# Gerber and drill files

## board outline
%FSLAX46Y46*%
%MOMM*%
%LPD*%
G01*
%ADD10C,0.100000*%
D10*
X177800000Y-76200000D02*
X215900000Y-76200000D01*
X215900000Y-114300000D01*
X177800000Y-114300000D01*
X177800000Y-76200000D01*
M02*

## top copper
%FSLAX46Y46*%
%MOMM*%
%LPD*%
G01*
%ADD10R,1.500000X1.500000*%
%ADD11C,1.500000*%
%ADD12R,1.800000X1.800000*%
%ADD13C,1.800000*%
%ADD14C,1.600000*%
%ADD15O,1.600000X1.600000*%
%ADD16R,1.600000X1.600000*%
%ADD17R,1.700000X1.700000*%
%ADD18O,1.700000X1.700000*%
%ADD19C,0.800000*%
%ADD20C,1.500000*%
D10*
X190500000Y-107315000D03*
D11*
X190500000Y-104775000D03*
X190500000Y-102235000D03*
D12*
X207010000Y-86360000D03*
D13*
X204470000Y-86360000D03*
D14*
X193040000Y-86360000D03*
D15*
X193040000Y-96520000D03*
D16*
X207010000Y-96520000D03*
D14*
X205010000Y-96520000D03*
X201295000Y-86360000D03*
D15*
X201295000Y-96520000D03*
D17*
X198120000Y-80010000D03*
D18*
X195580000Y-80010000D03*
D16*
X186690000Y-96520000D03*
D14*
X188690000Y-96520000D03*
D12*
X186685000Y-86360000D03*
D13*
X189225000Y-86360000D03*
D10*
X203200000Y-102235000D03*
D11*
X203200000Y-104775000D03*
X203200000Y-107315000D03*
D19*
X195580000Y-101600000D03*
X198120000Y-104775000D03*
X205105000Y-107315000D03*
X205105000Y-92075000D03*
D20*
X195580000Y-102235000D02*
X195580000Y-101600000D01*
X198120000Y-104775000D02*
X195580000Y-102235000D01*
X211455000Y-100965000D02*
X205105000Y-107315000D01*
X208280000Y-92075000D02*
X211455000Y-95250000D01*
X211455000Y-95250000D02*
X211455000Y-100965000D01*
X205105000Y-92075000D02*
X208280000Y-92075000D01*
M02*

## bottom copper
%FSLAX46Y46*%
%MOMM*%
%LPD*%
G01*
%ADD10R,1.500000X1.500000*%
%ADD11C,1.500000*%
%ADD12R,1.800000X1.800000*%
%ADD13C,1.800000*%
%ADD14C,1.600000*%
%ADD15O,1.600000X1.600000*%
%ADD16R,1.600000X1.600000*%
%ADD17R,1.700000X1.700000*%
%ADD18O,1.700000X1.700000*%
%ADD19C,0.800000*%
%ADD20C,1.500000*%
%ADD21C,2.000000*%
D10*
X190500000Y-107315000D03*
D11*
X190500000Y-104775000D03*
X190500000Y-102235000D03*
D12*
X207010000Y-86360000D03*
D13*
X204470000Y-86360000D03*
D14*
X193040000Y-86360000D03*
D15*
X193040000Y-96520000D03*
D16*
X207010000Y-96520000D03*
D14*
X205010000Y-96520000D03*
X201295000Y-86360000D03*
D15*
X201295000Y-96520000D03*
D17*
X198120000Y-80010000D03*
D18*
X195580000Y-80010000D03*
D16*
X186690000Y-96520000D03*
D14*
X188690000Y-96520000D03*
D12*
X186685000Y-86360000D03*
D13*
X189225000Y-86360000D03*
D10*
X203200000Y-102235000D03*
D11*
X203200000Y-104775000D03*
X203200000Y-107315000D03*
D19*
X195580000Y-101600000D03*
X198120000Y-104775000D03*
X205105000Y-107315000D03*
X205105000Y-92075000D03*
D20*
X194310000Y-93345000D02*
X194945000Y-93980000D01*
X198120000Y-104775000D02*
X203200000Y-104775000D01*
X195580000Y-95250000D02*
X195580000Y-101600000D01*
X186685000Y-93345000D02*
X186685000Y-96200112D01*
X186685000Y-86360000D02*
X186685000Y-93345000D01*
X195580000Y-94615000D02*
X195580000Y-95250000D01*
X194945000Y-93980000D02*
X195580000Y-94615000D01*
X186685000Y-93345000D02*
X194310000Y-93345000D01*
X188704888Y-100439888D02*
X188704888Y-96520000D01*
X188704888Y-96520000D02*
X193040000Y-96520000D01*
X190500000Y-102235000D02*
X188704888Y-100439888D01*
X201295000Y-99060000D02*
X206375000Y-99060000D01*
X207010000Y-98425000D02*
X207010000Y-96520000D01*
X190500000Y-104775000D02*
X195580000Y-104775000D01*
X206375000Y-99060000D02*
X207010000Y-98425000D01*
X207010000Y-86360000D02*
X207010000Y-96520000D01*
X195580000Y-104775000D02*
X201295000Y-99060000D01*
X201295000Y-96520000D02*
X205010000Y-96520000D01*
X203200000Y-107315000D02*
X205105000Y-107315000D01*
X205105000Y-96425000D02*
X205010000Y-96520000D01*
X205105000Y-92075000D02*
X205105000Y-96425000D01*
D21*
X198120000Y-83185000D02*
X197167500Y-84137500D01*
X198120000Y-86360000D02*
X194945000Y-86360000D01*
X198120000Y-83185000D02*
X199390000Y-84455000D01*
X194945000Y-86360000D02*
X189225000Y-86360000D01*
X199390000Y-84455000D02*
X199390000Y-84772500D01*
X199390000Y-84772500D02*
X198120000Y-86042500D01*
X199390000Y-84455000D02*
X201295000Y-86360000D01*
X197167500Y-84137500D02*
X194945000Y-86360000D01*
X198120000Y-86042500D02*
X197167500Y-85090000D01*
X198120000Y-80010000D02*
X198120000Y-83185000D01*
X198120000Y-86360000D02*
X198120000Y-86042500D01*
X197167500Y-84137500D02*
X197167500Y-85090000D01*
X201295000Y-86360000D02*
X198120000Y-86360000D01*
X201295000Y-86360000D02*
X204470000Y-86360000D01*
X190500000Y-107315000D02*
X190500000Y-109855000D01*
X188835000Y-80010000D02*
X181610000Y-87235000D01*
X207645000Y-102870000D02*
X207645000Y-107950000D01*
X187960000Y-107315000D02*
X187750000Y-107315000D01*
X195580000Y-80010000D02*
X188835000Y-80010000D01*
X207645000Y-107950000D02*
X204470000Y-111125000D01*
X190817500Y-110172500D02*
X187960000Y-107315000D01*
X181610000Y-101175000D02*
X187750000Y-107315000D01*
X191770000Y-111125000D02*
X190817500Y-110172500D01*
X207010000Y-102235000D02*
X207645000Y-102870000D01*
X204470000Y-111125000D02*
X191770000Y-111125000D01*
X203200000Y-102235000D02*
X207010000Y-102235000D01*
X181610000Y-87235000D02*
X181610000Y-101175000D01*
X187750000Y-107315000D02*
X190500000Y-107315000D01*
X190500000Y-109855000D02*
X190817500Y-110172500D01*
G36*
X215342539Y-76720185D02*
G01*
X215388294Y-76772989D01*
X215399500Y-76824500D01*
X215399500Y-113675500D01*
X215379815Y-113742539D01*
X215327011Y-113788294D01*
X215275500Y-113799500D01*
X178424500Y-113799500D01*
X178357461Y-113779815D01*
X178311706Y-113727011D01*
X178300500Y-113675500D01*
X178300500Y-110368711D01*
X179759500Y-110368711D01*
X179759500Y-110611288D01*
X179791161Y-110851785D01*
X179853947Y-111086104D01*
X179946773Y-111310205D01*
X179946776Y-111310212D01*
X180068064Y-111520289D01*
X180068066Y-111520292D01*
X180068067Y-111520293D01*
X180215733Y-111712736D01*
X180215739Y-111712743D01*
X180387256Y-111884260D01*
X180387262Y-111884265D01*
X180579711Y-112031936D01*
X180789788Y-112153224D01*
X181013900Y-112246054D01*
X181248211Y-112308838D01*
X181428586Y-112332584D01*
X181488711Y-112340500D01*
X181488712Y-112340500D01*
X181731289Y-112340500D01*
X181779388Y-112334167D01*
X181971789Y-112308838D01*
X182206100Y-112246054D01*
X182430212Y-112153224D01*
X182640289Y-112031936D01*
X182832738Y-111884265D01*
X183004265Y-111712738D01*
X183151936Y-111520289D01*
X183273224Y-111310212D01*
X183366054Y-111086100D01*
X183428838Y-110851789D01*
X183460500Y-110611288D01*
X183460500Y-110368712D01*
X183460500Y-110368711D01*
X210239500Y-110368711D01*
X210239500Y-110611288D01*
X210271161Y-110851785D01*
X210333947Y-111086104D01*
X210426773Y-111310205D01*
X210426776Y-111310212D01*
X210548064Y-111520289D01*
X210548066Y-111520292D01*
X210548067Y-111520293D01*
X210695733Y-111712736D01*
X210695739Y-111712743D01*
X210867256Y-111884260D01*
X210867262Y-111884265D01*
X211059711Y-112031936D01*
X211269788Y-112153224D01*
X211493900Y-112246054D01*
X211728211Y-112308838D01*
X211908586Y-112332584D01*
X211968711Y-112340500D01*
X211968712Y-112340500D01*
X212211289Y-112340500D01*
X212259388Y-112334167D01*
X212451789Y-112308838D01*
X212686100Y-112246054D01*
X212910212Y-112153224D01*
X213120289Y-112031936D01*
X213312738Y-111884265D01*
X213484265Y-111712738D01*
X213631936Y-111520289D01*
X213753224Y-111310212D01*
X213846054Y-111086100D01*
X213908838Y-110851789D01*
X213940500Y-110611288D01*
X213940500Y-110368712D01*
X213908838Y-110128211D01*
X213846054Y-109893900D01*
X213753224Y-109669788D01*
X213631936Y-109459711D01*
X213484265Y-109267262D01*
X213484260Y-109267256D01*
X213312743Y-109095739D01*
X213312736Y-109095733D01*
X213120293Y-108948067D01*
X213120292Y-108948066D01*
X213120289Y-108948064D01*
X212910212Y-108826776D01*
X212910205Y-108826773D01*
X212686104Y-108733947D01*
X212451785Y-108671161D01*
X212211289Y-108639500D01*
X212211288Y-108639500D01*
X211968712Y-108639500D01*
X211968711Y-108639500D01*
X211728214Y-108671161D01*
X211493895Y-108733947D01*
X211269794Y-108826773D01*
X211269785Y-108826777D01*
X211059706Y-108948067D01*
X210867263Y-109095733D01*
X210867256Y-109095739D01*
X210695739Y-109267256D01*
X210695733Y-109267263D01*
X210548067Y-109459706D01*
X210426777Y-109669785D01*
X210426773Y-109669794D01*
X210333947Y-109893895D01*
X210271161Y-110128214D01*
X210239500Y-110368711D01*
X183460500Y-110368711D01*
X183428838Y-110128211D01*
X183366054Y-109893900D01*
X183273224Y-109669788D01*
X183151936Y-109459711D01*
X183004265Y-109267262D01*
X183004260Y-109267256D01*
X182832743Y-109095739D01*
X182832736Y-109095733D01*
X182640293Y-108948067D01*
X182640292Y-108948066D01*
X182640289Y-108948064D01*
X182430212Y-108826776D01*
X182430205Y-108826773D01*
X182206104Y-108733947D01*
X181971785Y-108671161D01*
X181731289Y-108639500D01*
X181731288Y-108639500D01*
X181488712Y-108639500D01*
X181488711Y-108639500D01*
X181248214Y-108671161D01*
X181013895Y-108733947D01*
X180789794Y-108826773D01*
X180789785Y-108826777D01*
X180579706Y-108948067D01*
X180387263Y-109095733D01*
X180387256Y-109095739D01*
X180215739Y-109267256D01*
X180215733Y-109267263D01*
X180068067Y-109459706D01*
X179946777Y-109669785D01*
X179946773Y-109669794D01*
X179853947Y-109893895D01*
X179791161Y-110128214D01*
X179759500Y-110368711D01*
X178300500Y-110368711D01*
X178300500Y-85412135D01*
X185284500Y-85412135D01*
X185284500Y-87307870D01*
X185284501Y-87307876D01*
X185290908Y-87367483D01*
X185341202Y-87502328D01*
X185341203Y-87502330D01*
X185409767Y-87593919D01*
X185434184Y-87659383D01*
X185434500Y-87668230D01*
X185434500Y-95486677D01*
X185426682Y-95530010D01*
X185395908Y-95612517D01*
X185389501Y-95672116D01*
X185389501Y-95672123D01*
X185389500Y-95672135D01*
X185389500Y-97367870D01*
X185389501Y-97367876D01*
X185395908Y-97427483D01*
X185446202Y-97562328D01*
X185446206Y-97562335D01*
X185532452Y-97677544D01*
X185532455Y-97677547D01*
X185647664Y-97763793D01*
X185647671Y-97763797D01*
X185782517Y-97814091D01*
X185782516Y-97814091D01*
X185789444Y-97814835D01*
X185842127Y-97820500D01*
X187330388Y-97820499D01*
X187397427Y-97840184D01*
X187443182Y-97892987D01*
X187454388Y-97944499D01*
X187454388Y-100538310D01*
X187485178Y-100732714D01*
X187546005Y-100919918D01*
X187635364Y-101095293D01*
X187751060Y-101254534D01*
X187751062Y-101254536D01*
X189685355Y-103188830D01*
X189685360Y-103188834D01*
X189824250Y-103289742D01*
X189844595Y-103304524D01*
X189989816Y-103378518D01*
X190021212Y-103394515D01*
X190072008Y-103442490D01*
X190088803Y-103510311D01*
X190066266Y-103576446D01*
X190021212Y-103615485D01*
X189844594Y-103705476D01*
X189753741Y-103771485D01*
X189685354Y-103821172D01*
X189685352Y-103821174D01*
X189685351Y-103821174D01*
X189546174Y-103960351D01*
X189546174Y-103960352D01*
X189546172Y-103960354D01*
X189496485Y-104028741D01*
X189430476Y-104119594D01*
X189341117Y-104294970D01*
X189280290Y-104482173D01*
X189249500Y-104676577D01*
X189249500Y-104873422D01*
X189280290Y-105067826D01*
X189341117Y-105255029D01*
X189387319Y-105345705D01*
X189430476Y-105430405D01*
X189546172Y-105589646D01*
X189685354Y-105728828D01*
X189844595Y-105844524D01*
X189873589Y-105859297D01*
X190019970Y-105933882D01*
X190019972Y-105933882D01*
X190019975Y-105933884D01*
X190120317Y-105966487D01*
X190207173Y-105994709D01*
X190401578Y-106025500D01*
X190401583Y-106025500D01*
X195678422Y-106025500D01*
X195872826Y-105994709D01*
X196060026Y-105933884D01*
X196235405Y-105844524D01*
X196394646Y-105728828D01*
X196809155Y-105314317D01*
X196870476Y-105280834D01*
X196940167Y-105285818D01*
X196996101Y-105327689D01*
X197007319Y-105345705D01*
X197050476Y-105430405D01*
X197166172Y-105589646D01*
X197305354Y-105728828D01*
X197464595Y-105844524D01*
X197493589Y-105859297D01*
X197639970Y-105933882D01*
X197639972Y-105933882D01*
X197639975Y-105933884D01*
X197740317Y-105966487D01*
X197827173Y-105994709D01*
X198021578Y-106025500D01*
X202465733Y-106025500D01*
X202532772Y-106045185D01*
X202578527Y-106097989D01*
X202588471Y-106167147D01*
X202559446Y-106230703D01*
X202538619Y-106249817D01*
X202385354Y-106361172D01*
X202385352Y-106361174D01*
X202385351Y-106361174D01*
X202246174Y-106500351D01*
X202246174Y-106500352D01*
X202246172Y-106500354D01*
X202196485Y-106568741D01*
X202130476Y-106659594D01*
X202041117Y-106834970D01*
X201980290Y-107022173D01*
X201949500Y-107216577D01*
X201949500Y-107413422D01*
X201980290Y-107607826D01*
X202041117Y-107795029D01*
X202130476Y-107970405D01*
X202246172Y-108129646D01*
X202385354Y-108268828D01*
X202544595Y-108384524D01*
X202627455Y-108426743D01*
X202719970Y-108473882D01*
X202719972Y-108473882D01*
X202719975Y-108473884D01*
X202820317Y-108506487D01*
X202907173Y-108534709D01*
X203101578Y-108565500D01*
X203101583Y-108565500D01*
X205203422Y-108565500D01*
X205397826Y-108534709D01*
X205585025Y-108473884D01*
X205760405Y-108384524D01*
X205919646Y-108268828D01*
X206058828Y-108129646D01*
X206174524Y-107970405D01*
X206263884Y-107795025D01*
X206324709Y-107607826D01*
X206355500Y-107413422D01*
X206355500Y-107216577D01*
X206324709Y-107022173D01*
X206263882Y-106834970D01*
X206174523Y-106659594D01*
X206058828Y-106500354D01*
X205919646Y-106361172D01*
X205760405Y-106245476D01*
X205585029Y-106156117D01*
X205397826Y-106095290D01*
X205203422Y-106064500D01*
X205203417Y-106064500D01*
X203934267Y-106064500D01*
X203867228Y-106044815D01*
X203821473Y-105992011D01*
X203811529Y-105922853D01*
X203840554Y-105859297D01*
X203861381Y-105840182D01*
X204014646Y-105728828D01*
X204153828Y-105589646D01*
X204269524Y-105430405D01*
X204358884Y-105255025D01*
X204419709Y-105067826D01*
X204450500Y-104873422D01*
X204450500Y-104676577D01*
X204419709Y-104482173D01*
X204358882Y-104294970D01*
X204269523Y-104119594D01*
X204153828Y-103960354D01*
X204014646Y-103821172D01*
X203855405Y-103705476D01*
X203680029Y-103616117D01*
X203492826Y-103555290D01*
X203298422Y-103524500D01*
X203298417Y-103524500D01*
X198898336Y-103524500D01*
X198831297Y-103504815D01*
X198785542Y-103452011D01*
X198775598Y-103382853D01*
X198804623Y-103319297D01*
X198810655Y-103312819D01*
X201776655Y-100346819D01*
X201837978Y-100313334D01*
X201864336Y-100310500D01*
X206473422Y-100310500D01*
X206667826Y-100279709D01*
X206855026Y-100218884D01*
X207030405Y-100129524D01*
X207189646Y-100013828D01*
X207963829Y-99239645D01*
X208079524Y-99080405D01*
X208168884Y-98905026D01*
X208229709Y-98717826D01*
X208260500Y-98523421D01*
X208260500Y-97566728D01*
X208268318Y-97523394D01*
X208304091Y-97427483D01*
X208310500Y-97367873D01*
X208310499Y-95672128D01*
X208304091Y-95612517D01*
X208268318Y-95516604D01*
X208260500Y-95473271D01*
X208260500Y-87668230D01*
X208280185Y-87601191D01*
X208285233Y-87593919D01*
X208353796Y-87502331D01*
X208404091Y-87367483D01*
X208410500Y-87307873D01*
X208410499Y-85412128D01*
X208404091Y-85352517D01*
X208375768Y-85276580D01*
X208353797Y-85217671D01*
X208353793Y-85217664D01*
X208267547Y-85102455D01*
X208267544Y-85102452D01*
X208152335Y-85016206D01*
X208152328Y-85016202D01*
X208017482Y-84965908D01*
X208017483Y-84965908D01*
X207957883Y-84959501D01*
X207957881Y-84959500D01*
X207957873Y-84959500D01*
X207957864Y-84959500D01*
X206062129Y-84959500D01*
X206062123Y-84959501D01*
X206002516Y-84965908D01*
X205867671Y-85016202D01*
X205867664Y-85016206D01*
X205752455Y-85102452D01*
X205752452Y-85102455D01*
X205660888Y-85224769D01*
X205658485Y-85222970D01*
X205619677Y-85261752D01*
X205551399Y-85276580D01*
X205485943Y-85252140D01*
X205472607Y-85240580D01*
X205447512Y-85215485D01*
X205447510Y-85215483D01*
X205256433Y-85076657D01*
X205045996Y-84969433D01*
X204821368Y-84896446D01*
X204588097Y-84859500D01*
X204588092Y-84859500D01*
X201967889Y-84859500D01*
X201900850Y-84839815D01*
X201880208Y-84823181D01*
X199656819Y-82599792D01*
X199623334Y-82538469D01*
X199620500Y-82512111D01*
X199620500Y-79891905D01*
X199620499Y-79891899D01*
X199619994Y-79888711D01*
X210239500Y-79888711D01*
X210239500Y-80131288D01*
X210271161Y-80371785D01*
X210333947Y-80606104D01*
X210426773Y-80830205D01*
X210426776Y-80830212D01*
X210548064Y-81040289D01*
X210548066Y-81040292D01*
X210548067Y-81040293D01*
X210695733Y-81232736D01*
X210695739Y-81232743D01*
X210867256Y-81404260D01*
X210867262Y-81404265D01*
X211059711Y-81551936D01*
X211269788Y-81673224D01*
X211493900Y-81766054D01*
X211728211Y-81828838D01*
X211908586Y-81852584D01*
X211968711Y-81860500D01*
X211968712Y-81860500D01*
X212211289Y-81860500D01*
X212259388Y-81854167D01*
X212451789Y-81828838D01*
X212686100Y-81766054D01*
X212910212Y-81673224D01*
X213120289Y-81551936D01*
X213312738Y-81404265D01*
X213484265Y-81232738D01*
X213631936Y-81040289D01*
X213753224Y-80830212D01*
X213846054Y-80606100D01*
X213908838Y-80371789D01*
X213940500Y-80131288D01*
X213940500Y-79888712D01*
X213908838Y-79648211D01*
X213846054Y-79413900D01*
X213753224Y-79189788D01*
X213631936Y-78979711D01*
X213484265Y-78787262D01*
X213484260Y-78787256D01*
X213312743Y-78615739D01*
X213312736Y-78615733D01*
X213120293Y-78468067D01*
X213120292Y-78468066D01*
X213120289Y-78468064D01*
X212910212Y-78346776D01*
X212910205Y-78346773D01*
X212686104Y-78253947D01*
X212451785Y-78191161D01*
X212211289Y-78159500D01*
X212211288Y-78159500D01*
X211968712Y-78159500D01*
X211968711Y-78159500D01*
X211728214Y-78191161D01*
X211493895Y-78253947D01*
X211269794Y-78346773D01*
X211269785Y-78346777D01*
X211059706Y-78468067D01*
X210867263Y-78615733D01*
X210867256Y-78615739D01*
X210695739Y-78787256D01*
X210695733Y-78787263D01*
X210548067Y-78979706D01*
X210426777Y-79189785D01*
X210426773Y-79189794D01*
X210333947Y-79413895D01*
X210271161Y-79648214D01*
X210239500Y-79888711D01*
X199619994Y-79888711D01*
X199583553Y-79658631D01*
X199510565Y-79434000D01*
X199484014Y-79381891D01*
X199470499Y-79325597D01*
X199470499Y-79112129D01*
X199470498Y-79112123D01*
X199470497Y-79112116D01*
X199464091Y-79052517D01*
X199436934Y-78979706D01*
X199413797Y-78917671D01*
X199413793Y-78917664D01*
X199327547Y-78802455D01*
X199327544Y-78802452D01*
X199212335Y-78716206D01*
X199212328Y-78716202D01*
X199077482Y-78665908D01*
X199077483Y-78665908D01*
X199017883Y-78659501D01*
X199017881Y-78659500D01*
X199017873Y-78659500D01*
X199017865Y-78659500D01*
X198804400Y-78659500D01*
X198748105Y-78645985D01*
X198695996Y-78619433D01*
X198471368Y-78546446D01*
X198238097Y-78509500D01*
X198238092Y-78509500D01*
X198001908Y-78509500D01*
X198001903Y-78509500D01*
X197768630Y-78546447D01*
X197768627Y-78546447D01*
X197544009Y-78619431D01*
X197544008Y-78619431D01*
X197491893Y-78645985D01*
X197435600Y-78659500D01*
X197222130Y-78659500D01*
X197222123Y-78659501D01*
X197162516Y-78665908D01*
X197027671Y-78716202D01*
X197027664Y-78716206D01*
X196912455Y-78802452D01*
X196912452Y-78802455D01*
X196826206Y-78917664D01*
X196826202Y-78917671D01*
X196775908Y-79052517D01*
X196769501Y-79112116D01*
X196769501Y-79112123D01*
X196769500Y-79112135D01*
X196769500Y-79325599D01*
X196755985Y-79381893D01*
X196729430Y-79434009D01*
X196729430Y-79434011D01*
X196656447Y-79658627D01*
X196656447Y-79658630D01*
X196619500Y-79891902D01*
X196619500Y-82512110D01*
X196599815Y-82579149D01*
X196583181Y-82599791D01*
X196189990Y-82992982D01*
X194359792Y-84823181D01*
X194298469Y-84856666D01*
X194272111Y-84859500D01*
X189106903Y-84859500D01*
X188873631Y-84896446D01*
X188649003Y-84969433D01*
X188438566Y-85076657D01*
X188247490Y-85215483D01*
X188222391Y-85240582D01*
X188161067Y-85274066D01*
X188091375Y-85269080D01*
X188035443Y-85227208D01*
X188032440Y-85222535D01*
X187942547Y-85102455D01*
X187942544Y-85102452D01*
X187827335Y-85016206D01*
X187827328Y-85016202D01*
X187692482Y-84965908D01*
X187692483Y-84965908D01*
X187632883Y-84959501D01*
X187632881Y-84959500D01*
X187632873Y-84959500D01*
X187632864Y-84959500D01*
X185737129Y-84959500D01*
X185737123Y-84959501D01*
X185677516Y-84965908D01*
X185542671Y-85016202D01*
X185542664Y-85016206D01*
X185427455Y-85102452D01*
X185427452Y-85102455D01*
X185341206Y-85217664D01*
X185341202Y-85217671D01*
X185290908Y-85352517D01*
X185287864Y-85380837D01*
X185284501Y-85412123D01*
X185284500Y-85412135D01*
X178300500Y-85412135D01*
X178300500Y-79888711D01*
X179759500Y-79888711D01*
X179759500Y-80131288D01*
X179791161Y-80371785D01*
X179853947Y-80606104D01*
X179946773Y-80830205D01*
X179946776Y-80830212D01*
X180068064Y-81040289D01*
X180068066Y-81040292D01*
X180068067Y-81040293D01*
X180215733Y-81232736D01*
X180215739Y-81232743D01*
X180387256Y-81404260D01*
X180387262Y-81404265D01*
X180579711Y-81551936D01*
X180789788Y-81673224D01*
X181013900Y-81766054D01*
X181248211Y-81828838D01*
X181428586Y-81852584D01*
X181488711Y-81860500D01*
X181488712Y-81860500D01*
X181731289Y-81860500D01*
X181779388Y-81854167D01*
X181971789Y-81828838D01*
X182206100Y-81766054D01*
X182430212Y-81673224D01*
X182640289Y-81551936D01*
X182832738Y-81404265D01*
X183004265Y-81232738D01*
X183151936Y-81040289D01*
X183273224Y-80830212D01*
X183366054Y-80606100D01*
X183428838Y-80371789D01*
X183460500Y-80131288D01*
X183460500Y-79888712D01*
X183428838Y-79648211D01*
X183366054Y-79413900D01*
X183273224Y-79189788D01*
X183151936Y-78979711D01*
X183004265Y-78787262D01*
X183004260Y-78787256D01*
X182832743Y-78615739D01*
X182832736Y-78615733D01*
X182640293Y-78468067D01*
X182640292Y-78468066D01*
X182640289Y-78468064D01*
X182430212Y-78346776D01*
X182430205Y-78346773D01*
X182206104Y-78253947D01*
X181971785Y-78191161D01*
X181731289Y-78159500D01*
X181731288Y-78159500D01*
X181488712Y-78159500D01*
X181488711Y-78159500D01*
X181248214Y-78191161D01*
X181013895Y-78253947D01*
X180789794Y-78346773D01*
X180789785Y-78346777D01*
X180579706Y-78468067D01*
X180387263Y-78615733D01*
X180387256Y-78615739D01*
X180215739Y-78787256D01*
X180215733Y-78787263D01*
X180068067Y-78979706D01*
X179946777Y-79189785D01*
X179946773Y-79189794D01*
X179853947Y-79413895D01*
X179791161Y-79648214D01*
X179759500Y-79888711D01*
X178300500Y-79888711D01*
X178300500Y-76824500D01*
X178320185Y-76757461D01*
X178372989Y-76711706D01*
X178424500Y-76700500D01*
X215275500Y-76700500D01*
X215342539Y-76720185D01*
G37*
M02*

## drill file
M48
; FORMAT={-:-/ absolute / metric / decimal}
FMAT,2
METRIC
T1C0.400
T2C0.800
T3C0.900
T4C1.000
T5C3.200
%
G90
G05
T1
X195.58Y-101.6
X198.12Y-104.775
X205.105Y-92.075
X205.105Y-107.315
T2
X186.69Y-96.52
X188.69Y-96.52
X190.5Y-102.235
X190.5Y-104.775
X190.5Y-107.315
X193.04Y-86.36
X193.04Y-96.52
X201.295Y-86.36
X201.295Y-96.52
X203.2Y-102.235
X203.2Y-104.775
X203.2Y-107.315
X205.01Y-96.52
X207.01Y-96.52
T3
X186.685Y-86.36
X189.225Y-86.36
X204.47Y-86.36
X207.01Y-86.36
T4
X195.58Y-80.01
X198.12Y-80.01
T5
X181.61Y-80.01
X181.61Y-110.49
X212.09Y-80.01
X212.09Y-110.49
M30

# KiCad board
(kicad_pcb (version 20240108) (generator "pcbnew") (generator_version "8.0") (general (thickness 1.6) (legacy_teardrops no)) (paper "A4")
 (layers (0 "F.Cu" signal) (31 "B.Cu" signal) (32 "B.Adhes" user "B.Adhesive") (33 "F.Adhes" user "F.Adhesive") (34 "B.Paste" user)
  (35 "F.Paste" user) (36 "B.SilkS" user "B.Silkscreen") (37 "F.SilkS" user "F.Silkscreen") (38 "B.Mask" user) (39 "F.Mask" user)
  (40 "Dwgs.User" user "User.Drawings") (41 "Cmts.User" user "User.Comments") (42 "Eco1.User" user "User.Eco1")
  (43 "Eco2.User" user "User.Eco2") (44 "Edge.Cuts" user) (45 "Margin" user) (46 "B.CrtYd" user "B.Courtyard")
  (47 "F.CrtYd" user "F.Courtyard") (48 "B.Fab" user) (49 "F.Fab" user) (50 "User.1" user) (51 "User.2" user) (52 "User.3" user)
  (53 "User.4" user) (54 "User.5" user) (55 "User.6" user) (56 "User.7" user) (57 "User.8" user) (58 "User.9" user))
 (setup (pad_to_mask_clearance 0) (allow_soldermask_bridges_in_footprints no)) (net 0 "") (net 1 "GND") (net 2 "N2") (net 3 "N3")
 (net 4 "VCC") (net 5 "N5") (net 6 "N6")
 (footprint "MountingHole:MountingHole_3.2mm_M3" (layer "F.Cu") (at 181.61 110.49)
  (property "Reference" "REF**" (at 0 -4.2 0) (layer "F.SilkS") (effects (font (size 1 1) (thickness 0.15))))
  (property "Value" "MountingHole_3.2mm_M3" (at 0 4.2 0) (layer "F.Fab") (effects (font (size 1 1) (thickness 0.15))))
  (pad "" np_thru_hole circle (at 0 0) (size 3.2 3.2) (drill 3.2) (layers "F&B.Cu" "*.Mask")))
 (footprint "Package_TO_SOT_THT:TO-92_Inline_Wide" (layer "F.Cu") (at 190.5 107.315 90)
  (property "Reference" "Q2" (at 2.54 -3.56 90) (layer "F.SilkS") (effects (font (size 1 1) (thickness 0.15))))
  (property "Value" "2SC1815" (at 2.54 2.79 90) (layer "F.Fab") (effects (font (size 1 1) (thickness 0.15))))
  (pad "1" thru_hole rect (at 0 0 90) (size 1.5 1.5) (drill 0.8) (layers "*.Cu" "*.Mask") (remove_unused_layers no) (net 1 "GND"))
  (pad "2" thru_hole circle (at 2.54 0 90) (size 1.5 1.5) (drill 0.8) (layers "*.Cu" "*.Mask") (remove_unused_layers no) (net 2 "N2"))
  (pad "3" thru_hole circle (at 5.08 0 90) (size 1.5 1.5) (drill 0.8) (layers "*.Cu" "*.Mask") (remove_unused_layers no) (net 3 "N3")))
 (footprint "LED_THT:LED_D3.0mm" (layer "F.Cu") (at 207.01 86.36 180)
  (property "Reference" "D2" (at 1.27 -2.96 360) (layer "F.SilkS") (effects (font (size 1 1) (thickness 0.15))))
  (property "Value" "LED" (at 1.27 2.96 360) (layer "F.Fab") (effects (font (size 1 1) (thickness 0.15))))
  (pad "1" thru_hole rect (at 0 0 180) (size 1.8 1.8) (drill 0.9) (layers "*.Cu" "*.Mask") (remove_unused_layers no) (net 2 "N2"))
  (pad "2" thru_hole circle (at 2.54 0 180) (size 1.8 1.8) (drill 0.9) (layers "*.Cu" "*.Mask") (remove_unused_layers no) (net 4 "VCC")))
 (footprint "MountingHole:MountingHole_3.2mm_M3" (layer "F.Cu") (at 212.09 110.49)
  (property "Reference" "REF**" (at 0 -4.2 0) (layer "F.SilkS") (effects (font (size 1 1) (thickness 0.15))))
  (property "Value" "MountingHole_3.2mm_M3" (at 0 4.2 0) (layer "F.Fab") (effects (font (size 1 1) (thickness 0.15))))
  (pad "" np_thru_hole circle (at 0 0) (size 3.2 3.2) (drill 3.2) (layers "F&B.Cu" "*.Mask")))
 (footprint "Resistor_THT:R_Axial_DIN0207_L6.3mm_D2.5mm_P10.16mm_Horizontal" (layer "F.Cu") (at 193.04 86.36 -90)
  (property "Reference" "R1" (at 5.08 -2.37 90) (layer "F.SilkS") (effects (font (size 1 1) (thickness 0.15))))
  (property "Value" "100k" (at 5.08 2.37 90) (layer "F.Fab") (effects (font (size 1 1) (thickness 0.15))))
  (pad "1" thru_hole circle (at 0 0 270) (size 1.6 1.6) (drill 0.8) (layers "*.Cu" "*.Mask") (remove_unused_layers no) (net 4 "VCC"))
  (pad "2" thru_hole oval (at 10.16 0 270) (size 1.6 1.6) (drill 0.8) (layers "*.Cu" "*.Mask") (remove_unused_layers no) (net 3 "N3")))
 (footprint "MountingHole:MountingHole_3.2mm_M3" (layer "F.Cu") (at 181.61 80.01)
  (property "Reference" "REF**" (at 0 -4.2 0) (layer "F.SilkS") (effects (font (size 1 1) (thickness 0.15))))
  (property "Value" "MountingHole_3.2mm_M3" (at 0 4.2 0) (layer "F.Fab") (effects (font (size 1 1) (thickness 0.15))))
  (pad "" np_thru_hole circle (at 0 0) (size 3.2 3.2) (drill 3.2) (layers "*.Cu" "*.Mask")))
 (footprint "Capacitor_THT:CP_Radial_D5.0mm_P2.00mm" (layer "F.Cu") (at 207.01 96.52 180)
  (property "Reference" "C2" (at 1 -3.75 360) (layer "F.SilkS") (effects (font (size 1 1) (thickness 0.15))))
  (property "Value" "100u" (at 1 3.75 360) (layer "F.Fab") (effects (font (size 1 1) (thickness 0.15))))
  (pad "1" thru_hole rect (at 0 0 180) (size 1.6 1.6) (drill 0.8) (layers "*.Cu" "*.Mask") (remove_unused_layers no) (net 2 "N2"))
  (pad "2" thru_hole circle (at 2 0 180) (size 1.6 1.6) (drill 0.8) (layers "*.Cu" "*.Mask") (remove_unused_layers no) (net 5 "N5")))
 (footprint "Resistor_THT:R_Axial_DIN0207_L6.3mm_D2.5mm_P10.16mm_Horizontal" (layer "F.Cu") (at 201.295 86.36 -90)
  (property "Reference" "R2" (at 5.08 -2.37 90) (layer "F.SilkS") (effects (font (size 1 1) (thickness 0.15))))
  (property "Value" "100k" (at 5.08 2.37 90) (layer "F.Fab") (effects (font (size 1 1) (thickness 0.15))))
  (pad "1" thru_hole circle (at 0 0 270) (size 1.6 1.6) (drill 0.8) (layers "*.Cu" "*.Mask") (remove_unused_layers no) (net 4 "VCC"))
  (pad "2" thru_hole oval (at 10.16 0 270) (size 1.6 1.6) (drill 0.8) (layers "*.Cu" "*.Mask") (remove_unused_layers no) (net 5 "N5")))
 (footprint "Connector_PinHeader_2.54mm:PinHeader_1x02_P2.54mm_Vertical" (layer "F.Cu") (at 198.12 80.01 -90)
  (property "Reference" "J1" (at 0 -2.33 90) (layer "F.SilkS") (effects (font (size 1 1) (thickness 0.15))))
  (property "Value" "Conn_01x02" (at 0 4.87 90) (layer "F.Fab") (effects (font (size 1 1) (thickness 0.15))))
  (pad "1" thru_hole rect (at 0 0 270) (size 1.7 1.7) (drill 1) (layers "*.Cu" "*.Mask") (remove_unused_layers no) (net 4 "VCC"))
  (pad "2" thru_hole oval (at 0 2.54 270) (size 1.7 1.7) (drill 1) (layers "*.Cu" "*.Mask") (remove_unused_layers no) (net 1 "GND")))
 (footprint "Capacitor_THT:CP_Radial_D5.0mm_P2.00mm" (layer "F.Cu") (at 186.69 96.52)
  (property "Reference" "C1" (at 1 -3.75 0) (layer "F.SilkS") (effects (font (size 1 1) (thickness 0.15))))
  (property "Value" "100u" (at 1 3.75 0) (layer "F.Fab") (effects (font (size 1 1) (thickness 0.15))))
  (pad "1" thru_hole rect (at 0 0) (size 1.6 1.6) (drill 0.8) (layers "*.Cu" "*.Mask") (remove_unused_layers no) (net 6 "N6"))
  (pad "2" thru_hole circle (at 2 0) (size 1.6 1.6) (drill 0.8) (layers "*.Cu" "*.Mask") (remove_unused_layers no) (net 3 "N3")))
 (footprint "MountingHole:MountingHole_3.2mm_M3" (layer "F.Cu") (at 212.09 80.01)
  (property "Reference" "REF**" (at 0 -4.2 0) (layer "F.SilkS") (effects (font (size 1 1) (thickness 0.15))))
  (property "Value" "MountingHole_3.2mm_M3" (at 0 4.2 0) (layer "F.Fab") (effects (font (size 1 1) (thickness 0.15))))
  (pad "" np_thru_hole circle (at 0 0) (size 3.2 3.2) (drill 3.2) (layers "F&B.Cu" "*.Mask")))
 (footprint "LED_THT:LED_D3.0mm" (layer "F.Cu") (at 186.685 86.36)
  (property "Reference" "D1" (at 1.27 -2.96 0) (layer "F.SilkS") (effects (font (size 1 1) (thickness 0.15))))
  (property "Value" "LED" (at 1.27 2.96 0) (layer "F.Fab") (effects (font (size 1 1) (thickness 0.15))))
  (pad "1" thru_hole rect (at 0 0) (size 1.8 1.8) (drill 0.9) (layers "*.Cu" "*.Mask") (remove_unused_layers no) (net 6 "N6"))
  (pad "2" thru_hole circle (at 2.54 0) (size 1.8 1.8) (drill 0.9) (layers "*.Cu" "*.Mask") (remove_unused_layers no) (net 4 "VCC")))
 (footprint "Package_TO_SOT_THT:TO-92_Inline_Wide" (layer "F.Cu") (at 203.2 102.235 -90)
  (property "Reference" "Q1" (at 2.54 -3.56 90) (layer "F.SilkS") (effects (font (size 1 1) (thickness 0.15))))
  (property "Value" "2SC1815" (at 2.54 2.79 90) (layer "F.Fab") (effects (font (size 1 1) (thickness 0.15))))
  (pad "1" thru_hole rect (at 0 0 270) (size 1.5 1.5) (drill 0.8) (layers "*.Cu" "*.Mask") (remove_unused_layers no) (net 1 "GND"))
  (pad "2" thru_hole circle (at 2.54 0 270) (size 1.5 1.5) (drill 0.8) (layers "*.Cu" "*.Mask") (remove_unused_layers no) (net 6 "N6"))
  (pad "3" thru_hole circle (at 5.08 0 270) (size 1.5 1.5) (drill 0.8) (layers "*.Cu" "*.Mask") (remove_unused_layers no) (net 5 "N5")))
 (gr_rect (start 177.8 76.2) (end 215.9 114.3) (stroke (width 0.1) (type default)) (fill none) (layer "Edge.Cuts"))
 (segment (start 195.58 102.235) (end 195.58 101.6) (width 1.5) (layer "F.Cu") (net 6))
 (segment (start 198.12 104.775) (end 195.58 102.235) (width 1.5) (layer "F.Cu") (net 6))
 (via (at 195.58 101.6) (size 0.8) (drill 0.4) (layers "F.Cu" "B.Cu") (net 6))
 (via (at 198.12 104.775) (size 0.8) (drill 0.4) (layers "F.Cu" "B.Cu") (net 6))
 (segment (start 194.31 93.345) (end 194.945 93.98) (width 1.5) (layer "B.Cu") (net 6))
 (segment (start 198.12 104.775) (end 203.2 104.775) (width 1.5) (layer "B.Cu") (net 6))
 (segment (start 195.58 95.25) (end 195.58 101.6) (width 1.5) (layer "B.Cu") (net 6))
 (segment (start 186.685 93.345) (end 186.685 96.200112) (width 1.5) (layer "B.Cu") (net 6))
 (segment (start 186.685 86.36) (end 186.685 93.345) (width 1.5) (layer "B.Cu") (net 6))
 (segment (start 195.58 94.615) (end 195.58 95.25) (width 1.5) (layer "B.Cu") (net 6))
 (segment (start 194.945 93.98) (end 195.58 94.615) (width 1.5) (layer "B.Cu") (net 6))
 (segment (start 186.685 93.345) (end 194.31 93.345) (width 1.5) (layer "B.Cu") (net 6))
 (segment (start 188.704888 100.439888) (end 188.704888 96.52) (width 1.5) (layer "B.Cu") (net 3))
 (segment (start 188.704888 96.52) (end 193.04 96.52) (width 1.5) (layer "B.Cu") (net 3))
 (segment (start 190.5 102.235) (end 188.704888 100.439888) (width 1.5) (layer "B.Cu") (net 3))
 (segment (start 201.295 99.06) (end 206.375 99.06) (width 1.5) (layer "B.Cu") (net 2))
 (segment (start 207.01 98.425) (end 207.01 96.52) (width 1.5) (layer "B.Cu") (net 2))
 (segment (start 190.5 104.775) (end 195.58 104.775) (width 1.5) (layer "B.Cu") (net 2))
 (segment (start 206.375 99.06) (end 207.01 98.425) (width 1.5) (layer "B.Cu") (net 2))
 (segment (start 207.01 86.36) (end 207.01 96.52) (width 1.5) (layer "B.Cu") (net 2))
 (segment (start 195.58 104.775) (end 201.295 99.06) (width 1.5) (layer "B.Cu") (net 2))
 (segment (start 211.455 100.965) (end 205.105 107.315) (width 1.5) (layer "F.Cu") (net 5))
 (segment (start 208.28 92.075) (end 211.455 95.25) (width 1.5) (layer "F.Cu") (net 5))
 (segment (start 211.455 95.25) (end 211.455 100.965) (width 1.5) (layer "F.Cu") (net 5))
 (segment (start 205.105 92.075) (end 208.28 92.075) (width 1.5) (layer "F.Cu") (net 5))
 (via (at 205.105 107.315) (size 0.8) (drill 0.4) (layers "F.Cu" "B.Cu") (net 5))
 (via (at 205.105 92.075) (size 0.8) (drill 0.4) (layers "F.Cu" "B.Cu") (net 5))
 (segment (start 201.295 96.52) (end 205.01 96.52) (width 1.5) (layer "B.Cu") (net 5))
 (segment (start 203.2 107.315) (end 205.105 107.315) (width 1.5) (layer "B.Cu") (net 5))
 (segment (start 205.105 96.425) (end 205.01 96.52) (width 1.5) (layer "B.Cu") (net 5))
 (segment (start 205.105 92.075) (end 205.105 96.425) (width 1.5) (layer "B.Cu") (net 5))
 (segment (start 198.12 83.185) (end 197.1675 84.1375) (width 2) (layer "B.Cu") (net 4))
 (segment (start 198.12 86.36) (end 194.945 86.36) (width 2) (layer "B.Cu") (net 4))
 (segment (start 198.12 83.185) (end 199.39 84.455) (width 2) (layer "B.Cu") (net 4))
 (segment (start 194.945 86.36) (end 189.225 86.36) (width 2) (layer "B.Cu") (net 4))
 (segment (start 199.39 84.455) (end 199.39 84.7725) (width 2) (layer "B.Cu") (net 4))
 (segment (start 199.39 84.7725) (end 198.12 86.0425) (width 2) (layer "B.Cu") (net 4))
 (segment (start 199.39 84.455) (end 201.295 86.36) (width 2) (layer "B.Cu") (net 4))
 (segment (start 197.1675 84.1375) (end 194.945 86.36) (width 2) (layer "B.Cu") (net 4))
 (segment (start 198.12 86.0425) (end 197.1675 85.09) (width 2) (layer "B.Cu") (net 4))
 (segment (start 198.12 80.01) (end 198.12 83.185) (width 2) (layer "B.Cu") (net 4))
 (segment (start 198.12 86.36) (end 198.12 86.0425) (width 2) (layer "B.Cu") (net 4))
 (segment (start 197.1675 84.1375) (end 197.1675 85.09) (width 2) (layer "B.Cu") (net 4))
 (segment (start 201.295 86.36) (end 198.12 86.36) (width 2) (layer "B.Cu") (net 4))
 (segment (start 201.295 86.36) (end 204.47 86.36) (width 2) (layer "B.Cu") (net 4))
 (segment (start 190.5 107.315) (end 190.5 109.855) (width 2) (layer "B.Cu") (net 1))
 (segment (start 188.835 80.01) (end 181.61 87.235) (width 2) (layer "B.Cu") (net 1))
 (segment (start 207.645 102.87) (end 207.645 107.95) (width 2) (layer "B.Cu") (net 1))
 (segment (start 187.96 107.315) (end 187.75 107.315) (width 2) (layer "B.Cu") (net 1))
 (segment (start 195.58 80.01) (end 188.835 80.01) (width 2) (layer "B.Cu") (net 1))
 (segment (start 207.645 107.95) (end 204.47 111.125) (width 2) (layer "B.Cu") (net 1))
 (segment (start 190.8175 110.1725) (end 187.96 107.315) (width 2) (layer "B.Cu") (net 1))
 (segment (start 181.61 101.175) (end 187.75 107.315) (width 2) (layer "B.Cu") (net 1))
 (segment (start 191.77 111.125) (end 190.8175 110.1725) (width 2) (layer "B.Cu") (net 1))
 (segment (start 207.01 102.235) (end 207.645 102.87) (width 2) (layer "B.Cu") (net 1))
 (segment (start 204.47 111.125) (end 191.77 111.125) (width 2) (layer "B.Cu") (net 1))
 (segment (start 203.2 102.235) (end 207.01 102.235) (width 2) (layer "B.Cu") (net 1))
 (segment (start 181.61 87.235) (end 181.61 101.175) (width 2) (layer "B.Cu") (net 1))
 (segment (start 187.75 107.315) (end 190.5 107.315) (width 2) (layer "B.Cu") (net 1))
 (segment (start 190.5 109.855) (end 190.8175 110.1725) (width 2) (layer "B.Cu") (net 1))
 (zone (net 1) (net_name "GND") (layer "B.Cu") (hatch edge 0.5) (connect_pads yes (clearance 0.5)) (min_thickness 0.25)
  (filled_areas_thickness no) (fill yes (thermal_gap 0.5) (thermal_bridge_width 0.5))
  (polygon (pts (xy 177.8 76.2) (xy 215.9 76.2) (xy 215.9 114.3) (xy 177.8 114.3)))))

